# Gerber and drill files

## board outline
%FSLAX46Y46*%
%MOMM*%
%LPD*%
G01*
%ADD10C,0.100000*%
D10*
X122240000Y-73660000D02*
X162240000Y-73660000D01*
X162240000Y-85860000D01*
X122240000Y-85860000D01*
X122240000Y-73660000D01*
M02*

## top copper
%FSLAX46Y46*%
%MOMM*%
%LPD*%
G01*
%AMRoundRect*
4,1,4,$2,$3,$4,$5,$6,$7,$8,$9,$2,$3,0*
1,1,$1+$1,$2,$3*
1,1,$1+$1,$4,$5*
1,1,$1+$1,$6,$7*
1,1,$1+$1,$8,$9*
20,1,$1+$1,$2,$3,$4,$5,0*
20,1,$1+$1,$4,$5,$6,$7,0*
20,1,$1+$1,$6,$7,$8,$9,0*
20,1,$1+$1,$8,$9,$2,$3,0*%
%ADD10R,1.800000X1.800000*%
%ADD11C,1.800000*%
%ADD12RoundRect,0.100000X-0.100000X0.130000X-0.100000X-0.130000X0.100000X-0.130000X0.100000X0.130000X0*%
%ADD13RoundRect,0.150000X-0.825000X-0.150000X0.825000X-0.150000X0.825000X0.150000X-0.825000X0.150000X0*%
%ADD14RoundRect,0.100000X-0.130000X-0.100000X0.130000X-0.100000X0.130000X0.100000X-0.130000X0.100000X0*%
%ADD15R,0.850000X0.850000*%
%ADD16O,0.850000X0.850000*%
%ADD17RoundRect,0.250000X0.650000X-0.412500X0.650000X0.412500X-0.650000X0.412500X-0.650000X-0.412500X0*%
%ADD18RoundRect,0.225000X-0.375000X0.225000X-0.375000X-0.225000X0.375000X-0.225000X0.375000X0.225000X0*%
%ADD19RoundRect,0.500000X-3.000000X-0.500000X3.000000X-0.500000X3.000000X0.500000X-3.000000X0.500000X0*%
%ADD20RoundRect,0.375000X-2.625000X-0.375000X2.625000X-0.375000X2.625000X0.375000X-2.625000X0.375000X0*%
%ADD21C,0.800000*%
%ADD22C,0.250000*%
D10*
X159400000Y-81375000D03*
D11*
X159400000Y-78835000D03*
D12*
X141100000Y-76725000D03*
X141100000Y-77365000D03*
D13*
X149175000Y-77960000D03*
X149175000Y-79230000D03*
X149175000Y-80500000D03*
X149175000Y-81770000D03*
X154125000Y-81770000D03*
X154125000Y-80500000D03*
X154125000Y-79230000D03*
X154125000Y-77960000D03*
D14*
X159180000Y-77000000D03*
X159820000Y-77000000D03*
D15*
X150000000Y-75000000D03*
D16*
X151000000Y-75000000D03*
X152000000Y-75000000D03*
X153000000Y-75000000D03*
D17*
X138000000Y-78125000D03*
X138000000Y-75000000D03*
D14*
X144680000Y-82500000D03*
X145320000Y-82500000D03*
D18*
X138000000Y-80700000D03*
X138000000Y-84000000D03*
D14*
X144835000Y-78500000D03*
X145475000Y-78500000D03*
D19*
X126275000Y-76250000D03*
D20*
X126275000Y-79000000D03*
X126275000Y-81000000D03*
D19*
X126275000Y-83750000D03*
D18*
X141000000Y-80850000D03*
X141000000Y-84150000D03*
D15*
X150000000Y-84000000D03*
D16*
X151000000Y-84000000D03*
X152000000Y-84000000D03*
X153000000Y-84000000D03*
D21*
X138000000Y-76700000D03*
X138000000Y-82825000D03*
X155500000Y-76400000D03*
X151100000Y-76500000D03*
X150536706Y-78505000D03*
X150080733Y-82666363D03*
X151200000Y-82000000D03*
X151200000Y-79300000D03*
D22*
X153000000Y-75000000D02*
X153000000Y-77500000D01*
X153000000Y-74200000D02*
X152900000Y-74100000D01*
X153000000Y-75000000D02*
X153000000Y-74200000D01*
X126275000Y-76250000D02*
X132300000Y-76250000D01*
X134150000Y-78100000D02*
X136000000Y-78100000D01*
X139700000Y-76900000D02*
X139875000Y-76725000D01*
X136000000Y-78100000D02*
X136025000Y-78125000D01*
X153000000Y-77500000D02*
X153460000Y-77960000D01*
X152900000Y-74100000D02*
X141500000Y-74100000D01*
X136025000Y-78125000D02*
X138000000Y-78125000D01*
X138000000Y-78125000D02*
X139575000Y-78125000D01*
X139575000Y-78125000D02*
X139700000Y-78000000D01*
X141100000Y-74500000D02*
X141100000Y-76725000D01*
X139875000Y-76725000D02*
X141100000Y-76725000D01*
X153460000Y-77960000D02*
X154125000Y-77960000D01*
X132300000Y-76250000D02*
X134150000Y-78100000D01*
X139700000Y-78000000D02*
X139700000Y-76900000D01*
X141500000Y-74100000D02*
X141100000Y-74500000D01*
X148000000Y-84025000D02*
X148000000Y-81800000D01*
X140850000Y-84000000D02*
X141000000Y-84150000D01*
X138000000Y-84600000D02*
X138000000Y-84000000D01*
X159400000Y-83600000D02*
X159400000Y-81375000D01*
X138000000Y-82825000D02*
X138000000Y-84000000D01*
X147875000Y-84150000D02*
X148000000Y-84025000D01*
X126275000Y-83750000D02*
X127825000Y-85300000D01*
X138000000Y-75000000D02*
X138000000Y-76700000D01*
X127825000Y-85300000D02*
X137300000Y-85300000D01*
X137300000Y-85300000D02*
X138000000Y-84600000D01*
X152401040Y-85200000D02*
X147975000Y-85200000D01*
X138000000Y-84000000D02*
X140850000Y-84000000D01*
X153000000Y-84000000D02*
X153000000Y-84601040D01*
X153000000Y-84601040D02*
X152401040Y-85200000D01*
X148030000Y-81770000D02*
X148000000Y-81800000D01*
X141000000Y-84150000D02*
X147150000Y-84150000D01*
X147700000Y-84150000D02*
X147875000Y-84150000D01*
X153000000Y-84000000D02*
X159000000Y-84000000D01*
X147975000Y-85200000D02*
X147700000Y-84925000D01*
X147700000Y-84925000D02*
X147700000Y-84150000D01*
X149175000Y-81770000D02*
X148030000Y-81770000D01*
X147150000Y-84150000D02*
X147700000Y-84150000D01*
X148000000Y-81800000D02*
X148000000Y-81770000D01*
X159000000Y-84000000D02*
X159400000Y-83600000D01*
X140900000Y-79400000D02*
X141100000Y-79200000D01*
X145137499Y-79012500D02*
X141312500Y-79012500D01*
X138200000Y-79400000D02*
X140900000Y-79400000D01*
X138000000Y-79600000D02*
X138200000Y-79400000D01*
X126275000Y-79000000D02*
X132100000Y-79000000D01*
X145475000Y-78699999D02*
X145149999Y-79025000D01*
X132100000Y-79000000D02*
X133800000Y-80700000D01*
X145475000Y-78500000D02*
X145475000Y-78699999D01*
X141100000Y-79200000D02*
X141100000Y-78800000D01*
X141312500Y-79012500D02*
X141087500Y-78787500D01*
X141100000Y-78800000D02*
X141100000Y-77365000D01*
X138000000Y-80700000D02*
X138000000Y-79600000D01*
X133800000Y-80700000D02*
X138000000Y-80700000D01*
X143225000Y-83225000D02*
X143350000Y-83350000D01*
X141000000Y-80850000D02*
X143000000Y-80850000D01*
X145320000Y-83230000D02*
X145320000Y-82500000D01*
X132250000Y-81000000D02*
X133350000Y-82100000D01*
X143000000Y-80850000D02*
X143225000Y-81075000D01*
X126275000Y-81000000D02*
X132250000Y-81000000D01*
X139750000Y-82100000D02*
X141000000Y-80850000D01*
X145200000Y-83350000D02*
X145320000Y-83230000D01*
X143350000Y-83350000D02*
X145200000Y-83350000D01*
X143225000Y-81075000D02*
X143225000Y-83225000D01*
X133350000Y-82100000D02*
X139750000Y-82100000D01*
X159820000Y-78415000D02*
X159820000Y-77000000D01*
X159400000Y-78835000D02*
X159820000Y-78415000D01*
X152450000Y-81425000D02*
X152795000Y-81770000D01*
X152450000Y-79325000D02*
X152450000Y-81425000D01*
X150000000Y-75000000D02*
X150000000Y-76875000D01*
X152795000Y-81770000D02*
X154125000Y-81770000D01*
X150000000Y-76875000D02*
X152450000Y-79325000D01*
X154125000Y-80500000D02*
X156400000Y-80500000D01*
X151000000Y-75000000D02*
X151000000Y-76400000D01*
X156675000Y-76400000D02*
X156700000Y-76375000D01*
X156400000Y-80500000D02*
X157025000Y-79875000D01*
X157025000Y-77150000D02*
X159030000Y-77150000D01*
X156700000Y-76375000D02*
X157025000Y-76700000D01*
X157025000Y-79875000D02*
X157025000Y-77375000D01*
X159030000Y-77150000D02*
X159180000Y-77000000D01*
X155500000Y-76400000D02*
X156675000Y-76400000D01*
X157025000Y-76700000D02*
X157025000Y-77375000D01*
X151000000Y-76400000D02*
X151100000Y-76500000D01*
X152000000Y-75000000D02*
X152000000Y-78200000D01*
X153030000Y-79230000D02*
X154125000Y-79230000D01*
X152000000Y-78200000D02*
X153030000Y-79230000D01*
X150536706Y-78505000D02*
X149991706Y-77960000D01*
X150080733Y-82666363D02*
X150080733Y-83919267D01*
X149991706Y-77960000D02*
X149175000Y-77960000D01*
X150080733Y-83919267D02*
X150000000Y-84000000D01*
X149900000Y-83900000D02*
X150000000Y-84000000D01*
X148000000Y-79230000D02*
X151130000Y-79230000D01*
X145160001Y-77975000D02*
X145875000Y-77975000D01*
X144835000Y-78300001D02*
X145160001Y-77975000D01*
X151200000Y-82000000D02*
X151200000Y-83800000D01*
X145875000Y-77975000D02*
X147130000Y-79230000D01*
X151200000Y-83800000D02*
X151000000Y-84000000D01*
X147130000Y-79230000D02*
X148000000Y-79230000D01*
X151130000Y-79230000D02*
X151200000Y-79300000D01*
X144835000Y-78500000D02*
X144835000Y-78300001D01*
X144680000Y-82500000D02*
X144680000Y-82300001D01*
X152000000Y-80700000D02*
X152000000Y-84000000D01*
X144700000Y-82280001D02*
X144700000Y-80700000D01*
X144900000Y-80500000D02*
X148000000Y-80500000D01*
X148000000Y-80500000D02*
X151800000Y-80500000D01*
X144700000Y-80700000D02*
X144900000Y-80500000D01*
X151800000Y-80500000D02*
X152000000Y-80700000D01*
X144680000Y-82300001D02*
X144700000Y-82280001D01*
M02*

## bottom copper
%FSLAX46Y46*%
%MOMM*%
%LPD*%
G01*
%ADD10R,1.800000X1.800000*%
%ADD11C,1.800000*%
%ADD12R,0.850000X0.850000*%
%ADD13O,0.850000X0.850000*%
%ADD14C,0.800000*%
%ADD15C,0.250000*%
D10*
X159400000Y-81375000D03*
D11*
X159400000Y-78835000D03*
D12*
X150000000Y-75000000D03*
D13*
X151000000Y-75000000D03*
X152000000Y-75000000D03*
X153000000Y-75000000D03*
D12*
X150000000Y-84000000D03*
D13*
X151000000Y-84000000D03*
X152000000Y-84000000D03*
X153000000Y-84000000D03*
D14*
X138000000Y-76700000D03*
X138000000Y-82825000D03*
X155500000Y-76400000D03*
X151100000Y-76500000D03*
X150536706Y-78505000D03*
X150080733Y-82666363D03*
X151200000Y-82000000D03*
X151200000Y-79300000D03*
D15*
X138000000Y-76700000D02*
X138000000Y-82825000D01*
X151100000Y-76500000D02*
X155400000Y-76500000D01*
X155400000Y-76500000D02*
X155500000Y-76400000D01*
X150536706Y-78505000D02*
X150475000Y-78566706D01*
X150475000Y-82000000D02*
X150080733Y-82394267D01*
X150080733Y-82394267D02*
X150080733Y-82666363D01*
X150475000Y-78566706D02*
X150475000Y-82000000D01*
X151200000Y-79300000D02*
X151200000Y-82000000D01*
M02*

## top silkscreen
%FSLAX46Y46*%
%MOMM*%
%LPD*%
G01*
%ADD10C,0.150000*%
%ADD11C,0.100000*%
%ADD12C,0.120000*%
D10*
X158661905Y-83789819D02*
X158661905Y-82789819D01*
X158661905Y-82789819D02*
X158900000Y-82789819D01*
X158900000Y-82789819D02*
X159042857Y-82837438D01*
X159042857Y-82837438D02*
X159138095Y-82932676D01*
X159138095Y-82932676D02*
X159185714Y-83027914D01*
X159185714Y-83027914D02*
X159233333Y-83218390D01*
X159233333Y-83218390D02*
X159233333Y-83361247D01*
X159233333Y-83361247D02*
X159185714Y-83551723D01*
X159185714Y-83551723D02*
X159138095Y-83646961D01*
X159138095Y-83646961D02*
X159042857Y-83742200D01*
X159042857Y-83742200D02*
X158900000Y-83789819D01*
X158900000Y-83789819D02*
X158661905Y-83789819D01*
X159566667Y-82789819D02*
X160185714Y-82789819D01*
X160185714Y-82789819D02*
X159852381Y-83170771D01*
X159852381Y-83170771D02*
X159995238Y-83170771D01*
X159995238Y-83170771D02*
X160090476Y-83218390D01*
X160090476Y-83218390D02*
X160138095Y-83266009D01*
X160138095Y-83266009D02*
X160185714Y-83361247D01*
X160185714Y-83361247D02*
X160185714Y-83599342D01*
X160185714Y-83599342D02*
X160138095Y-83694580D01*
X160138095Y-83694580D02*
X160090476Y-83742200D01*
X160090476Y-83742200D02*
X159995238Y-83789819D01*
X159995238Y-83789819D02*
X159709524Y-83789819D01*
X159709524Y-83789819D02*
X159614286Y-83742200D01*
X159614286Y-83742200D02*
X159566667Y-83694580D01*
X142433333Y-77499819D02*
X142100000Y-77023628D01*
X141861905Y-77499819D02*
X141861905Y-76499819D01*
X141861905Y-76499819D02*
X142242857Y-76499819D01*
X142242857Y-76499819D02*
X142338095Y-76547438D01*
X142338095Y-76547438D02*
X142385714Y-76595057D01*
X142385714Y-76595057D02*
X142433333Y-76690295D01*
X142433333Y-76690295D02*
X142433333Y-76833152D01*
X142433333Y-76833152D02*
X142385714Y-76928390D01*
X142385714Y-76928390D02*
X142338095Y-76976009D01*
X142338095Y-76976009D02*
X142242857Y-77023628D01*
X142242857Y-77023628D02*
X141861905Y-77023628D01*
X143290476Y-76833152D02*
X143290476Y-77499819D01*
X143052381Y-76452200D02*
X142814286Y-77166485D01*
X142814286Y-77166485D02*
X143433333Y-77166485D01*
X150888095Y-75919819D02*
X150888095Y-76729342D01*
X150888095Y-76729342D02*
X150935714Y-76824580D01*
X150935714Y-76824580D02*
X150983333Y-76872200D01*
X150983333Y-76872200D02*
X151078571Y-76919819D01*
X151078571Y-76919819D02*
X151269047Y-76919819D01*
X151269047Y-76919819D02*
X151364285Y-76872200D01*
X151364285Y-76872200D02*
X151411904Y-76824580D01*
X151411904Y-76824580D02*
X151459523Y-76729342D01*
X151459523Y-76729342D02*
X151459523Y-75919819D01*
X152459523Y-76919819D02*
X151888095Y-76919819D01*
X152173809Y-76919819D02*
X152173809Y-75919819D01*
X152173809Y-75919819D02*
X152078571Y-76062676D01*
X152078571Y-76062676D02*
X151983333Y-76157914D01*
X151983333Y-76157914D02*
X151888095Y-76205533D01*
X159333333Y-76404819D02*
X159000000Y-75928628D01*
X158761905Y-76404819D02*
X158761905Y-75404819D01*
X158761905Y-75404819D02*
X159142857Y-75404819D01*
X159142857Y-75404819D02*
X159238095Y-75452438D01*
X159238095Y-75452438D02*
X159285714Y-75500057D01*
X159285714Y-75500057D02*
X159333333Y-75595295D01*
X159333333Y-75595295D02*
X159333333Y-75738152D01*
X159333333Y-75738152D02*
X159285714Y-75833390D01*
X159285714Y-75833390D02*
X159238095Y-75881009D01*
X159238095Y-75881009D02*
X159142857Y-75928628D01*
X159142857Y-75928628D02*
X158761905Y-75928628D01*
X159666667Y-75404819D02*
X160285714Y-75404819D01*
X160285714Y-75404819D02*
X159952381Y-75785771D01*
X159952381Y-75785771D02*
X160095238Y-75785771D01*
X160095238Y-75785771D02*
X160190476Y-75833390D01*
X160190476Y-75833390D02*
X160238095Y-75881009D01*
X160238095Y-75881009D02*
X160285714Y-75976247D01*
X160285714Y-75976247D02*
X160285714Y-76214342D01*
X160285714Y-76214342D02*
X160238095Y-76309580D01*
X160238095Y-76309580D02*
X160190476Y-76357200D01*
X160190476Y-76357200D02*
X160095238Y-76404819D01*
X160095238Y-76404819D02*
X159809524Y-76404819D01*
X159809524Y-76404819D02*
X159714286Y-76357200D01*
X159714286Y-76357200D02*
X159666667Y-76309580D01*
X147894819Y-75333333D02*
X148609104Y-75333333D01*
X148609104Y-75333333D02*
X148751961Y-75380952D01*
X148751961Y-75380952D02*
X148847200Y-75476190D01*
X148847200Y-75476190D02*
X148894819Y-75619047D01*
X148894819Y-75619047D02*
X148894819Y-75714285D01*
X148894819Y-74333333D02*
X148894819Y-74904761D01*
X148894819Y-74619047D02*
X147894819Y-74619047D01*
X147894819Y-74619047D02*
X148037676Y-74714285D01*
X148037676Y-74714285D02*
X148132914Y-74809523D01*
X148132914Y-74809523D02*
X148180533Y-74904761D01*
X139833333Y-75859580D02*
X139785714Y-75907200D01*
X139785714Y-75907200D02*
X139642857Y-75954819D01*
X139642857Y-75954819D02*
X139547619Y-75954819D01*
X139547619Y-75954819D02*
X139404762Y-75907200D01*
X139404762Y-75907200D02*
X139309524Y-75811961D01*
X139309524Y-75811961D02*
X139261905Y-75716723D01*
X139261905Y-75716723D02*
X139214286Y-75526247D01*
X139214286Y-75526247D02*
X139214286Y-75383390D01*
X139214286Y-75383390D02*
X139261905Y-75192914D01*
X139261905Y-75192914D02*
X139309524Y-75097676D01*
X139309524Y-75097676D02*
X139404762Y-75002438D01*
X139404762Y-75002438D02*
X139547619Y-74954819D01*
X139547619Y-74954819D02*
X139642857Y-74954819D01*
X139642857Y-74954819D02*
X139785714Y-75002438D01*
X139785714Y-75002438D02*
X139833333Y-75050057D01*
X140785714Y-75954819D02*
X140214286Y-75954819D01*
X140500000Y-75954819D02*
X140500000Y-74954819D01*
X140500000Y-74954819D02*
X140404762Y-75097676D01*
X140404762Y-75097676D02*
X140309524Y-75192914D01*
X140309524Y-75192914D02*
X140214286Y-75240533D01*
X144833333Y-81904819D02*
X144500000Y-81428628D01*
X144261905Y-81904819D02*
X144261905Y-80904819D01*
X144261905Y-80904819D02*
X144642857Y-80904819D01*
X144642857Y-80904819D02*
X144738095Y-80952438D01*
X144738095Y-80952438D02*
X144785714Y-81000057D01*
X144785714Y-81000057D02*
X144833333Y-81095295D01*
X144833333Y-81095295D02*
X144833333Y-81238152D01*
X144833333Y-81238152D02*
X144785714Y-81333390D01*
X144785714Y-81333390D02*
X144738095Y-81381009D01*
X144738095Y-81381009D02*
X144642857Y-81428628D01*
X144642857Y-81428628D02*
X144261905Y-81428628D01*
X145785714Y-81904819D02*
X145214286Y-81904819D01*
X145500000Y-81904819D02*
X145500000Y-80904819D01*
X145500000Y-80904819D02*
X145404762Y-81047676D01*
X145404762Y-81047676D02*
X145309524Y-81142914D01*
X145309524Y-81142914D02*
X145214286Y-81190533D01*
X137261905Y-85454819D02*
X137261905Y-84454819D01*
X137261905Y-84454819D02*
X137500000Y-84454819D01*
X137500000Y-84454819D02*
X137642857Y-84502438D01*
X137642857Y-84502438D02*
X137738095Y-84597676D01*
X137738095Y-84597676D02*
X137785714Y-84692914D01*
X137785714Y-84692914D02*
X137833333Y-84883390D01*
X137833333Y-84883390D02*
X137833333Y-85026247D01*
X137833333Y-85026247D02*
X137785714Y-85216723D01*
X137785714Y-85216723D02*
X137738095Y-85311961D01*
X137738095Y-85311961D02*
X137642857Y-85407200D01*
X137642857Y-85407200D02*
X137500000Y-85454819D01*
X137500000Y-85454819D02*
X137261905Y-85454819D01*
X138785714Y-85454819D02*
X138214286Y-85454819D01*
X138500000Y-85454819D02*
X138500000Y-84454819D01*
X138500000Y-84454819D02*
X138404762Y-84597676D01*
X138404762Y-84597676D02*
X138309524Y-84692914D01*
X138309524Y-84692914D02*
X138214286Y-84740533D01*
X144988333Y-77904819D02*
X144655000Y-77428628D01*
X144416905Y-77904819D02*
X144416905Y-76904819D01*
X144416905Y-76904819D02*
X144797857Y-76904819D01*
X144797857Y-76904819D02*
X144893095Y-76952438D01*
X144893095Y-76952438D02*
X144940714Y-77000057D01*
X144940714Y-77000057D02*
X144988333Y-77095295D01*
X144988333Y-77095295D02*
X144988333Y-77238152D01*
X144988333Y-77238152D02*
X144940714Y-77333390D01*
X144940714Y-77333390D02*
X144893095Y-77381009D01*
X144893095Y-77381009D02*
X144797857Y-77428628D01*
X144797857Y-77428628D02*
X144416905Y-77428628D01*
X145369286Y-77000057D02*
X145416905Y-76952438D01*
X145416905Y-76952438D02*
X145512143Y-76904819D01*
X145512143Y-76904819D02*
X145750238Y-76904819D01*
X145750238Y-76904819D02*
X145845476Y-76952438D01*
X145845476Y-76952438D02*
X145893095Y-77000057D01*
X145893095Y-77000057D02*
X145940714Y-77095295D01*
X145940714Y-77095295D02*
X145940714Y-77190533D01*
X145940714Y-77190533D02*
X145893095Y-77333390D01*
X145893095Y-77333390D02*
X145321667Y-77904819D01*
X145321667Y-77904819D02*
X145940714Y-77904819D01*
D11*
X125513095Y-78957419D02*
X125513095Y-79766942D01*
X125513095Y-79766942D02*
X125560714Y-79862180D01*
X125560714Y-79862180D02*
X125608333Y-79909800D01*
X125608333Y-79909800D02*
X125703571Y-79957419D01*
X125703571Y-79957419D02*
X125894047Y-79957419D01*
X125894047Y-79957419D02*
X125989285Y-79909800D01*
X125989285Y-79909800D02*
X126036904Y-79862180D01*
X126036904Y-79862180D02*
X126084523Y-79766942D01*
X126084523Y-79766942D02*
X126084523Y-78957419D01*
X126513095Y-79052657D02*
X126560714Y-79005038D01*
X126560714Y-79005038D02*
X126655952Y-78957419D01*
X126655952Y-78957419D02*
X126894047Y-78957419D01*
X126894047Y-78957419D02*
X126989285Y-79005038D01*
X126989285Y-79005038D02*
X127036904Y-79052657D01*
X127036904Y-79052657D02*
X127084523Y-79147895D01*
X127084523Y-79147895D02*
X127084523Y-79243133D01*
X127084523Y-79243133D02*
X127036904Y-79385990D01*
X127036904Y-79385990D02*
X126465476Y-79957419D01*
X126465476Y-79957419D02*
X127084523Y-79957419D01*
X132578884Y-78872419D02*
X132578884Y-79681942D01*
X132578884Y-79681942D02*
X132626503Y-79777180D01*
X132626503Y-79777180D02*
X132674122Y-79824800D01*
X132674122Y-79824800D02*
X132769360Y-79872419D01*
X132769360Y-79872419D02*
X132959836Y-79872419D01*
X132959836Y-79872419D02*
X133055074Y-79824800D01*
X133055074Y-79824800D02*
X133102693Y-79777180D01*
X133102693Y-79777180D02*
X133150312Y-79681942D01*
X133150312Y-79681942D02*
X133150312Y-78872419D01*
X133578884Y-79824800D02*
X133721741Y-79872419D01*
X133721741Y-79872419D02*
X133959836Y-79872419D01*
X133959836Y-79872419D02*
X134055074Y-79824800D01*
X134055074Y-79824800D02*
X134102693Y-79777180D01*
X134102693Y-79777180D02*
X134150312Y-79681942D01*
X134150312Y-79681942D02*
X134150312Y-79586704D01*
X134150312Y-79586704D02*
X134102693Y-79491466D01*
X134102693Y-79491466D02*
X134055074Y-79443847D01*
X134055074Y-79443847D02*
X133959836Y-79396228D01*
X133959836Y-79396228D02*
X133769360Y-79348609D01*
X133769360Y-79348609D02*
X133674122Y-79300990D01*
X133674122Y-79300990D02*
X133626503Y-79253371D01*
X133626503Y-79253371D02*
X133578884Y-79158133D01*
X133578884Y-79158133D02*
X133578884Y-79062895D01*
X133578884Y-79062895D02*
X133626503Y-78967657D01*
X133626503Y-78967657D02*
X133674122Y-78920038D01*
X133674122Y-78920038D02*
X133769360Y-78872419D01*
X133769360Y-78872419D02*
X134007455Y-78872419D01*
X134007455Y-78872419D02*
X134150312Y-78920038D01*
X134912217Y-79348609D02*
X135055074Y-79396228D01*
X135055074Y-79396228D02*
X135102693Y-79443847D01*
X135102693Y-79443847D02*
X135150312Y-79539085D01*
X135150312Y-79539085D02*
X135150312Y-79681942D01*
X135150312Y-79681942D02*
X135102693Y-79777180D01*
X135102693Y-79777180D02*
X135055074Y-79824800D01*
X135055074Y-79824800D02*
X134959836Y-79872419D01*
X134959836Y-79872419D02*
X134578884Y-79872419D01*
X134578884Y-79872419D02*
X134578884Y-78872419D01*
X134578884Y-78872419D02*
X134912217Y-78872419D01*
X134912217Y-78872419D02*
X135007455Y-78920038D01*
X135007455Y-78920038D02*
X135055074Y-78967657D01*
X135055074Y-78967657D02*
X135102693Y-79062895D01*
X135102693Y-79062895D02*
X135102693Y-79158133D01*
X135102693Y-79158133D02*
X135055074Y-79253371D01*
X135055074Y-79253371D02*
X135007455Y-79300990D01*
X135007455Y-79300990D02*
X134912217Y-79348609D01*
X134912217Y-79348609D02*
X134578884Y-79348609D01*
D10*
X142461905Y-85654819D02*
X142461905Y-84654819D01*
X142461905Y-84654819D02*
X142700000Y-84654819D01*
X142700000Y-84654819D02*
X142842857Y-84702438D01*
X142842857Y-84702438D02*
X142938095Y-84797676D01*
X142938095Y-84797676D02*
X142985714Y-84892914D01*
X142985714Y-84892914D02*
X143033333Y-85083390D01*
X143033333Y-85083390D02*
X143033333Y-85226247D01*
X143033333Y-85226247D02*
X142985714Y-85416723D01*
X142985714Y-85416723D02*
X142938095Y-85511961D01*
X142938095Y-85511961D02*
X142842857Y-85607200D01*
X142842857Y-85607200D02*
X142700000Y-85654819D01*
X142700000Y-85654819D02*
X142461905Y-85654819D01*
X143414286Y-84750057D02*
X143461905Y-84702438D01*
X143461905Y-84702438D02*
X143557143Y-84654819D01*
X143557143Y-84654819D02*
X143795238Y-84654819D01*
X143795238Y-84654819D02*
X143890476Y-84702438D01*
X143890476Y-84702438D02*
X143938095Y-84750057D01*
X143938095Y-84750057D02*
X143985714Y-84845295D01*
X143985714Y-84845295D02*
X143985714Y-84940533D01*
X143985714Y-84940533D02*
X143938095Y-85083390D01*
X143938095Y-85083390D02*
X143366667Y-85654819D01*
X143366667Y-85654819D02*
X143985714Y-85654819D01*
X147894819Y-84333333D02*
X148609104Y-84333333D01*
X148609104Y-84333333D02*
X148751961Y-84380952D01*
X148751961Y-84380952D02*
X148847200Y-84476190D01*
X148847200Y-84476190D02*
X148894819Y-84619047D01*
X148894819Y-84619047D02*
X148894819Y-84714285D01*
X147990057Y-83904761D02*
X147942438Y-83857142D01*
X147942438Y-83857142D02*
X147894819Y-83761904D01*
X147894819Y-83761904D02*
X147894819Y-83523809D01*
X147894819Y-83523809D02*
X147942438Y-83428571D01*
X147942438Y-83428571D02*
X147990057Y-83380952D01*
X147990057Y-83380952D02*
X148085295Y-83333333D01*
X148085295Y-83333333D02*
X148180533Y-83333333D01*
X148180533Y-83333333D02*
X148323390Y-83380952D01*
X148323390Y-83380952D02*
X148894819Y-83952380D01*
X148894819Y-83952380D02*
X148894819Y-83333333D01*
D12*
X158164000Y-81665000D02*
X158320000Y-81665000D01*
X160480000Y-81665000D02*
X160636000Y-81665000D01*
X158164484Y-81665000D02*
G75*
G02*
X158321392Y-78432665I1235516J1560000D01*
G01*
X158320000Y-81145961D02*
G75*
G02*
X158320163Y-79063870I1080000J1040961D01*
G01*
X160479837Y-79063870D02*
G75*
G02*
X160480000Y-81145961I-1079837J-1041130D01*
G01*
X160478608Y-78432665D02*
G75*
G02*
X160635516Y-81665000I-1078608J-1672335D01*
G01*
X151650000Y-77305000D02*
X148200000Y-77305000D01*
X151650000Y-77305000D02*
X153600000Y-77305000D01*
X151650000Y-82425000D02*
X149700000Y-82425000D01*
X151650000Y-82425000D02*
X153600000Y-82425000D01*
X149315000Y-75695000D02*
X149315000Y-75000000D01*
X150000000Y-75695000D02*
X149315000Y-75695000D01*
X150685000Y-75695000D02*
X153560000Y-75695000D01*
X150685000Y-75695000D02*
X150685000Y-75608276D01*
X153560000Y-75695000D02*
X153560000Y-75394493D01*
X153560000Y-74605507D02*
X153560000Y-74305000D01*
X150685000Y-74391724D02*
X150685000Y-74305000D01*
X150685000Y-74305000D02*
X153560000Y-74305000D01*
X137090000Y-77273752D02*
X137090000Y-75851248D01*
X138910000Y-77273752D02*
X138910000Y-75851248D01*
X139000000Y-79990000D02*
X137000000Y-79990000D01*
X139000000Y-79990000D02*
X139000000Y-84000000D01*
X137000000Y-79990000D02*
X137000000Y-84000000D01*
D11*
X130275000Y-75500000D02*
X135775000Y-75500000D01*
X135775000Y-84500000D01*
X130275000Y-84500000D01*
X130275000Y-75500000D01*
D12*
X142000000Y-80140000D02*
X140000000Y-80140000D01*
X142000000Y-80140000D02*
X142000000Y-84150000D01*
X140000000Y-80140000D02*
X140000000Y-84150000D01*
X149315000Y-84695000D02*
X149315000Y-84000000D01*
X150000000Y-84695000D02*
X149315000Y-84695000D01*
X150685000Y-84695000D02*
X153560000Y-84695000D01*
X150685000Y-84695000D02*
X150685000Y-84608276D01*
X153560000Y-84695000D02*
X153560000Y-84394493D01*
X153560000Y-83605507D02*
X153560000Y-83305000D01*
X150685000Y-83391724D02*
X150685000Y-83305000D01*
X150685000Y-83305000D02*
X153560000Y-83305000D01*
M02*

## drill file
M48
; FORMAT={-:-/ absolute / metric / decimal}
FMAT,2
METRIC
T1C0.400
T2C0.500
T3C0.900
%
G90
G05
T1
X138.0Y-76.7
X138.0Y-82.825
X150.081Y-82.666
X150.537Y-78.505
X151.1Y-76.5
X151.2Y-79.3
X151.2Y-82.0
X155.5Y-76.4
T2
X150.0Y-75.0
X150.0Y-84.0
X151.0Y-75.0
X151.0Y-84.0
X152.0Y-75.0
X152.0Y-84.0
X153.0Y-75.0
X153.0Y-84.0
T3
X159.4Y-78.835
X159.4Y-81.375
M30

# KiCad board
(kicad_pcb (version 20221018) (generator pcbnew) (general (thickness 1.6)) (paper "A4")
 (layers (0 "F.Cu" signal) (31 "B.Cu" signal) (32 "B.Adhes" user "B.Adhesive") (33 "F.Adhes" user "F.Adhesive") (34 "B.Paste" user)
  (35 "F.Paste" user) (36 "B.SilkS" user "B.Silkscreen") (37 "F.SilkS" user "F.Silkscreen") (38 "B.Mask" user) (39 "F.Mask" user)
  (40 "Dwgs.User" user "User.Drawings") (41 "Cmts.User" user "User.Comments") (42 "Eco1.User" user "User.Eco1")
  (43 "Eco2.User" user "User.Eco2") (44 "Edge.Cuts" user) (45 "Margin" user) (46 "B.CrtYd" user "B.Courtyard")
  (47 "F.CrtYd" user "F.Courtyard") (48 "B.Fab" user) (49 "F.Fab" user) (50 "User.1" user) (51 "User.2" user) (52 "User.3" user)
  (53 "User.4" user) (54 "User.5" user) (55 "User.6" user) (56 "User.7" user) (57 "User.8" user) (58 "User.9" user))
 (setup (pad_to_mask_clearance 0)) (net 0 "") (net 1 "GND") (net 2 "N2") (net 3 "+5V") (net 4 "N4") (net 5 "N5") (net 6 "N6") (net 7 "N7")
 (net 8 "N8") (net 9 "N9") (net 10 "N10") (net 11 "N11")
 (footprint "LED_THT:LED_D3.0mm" (layer "F.Cu") (at 159.4 81.375 90)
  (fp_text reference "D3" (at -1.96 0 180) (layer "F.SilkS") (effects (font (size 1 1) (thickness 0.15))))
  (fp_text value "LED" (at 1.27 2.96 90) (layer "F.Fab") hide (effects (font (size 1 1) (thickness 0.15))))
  (fp_line (start -0.29 -1.236) (end -0.29 -1.08) (stroke (width 0.12) (type solid)) (layer "F.SilkS"))
  (fp_line (start -0.29 1.08) (end -0.29 1.236) (stroke (width 0.12) (type solid)) (layer "F.SilkS"))
  (fp_arc (start -0.29 -1.235516) (mid 1.366487 -1.987659) (end 2.942335 -1.078608) (stroke (width 0.12) (type solid)) (layer "F.SilkS"))
  (fp_arc (start 0.229039 -1.08) (mid 1.270117 -1.5) (end 2.31113 -1.079837) (stroke (width 0.12) (type solid)) (layer "F.SilkS"))
  (fp_arc (start 2.31113 1.079837) (mid 1.270117 1.5) (end 0.229039 1.08) (stroke (width 0.12) (type solid)) (layer "F.SilkS"))
  (fp_arc (start 2.942335 1.078608) (mid 1.366487 1.987659) (end -0.29 1.235516) (stroke (width 0.12) (type solid)) (layer "F.SilkS"))
  (pad "1" thru_hole rect (at 0 0 90) (size 1.8 1.8) (drill 0.9) (layers "*.Cu" "*.Mask") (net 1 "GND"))
  (pad "2" thru_hole circle (at 2.54 0 90) (size 1.8 1.8) (drill 0.9) (layers "*.Cu" "*.Mask") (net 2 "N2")))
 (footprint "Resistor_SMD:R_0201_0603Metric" (layer "F.Cu") (at 141.1 77.045 -90)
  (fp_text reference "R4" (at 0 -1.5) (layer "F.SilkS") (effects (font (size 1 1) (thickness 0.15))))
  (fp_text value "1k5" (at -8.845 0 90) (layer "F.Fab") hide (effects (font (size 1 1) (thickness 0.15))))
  (pad "" smd roundrect (at -0.345 0 270) (size 0.318 0.36) (layers "F.Paste") (roundrect_rratio 0.25))
  (pad "" smd roundrect (at 0.345 0 270) (size 0.318 0.36) (layers "F.Paste") (roundrect_rratio 0.25))
  (pad "1" smd roundrect (at -0.32 0 270) (size 0.46 0.4) (layers "F.Cu" "F.Mask") (roundrect_rratio 0.25) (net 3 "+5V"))
  (pad "2" smd roundrect (at 0.32 0 270) (size 0.46 0.4) (layers "F.Cu" "F.Mask") (roundrect_rratio 0.25) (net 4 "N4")))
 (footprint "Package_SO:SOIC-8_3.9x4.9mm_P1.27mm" (layer "F.Cu") (at 151.65 79.865)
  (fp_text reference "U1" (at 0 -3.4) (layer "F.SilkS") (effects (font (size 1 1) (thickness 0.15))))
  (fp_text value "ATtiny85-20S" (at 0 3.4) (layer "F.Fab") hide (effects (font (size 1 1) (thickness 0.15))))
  (fp_line (start 0 -2.56) (end -3.45 -2.56) (stroke (width 0.12) (type solid)) (layer "F.SilkS"))
  (fp_line (start 0 -2.56) (end 1.95 -2.56) (stroke (width 0.12) (type solid)) (layer "F.SilkS"))
  (fp_line (start 0 2.56) (end -1.95 2.56) (stroke (width 0.12) (type solid)) (layer "F.SilkS"))
  (fp_line (start 0 2.56) (end 1.95 2.56) (stroke (width 0.12) (type solid)) (layer "F.SilkS"))
  (pad "1" smd roundrect (at -2.475 -1.905) (size 1.95 0.6) (layers "F.Cu" "F.Paste" "F.Mask") (roundrect_rratio 0.25) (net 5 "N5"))
  (pad "2" smd roundrect (at -2.475 -0.635) (size 1.95 0.6) (layers "F.Cu" "F.Paste" "F.Mask") (roundrect_rratio 0.25) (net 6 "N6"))
  (pad "3" smd roundrect (at -2.475 0.635) (size 1.95 0.6) (layers "F.Cu" "F.Paste" "F.Mask") (roundrect_rratio 0.25) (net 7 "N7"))
  (pad "4" smd roundrect (at -2.475 1.905) (size 1.95 0.6) (layers "F.Cu" "F.Paste" "F.Mask") (roundrect_rratio 0.25) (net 1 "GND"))
  (pad "5" smd roundrect (at 2.475 1.905) (size 1.95 0.6) (layers "F.Cu" "F.Paste" "F.Mask") (roundrect_rratio 0.25) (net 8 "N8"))
  (pad "6" smd roundrect (at 2.475 0.635) (size 1.95 0.6) (layers "F.Cu" "F.Paste" "F.Mask") (roundrect_rratio 0.25) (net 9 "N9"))
  (pad "7" smd roundrect (at 2.475 -0.635) (size 1.95 0.6) (layers "F.Cu" "F.Paste" "F.Mask") (roundrect_rratio 0.25) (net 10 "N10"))
  (pad "8" smd roundrect (at 2.475 -1.905) (size 1.95 0.6) (layers "F.Cu" "F.Paste" "F.Mask") (roundrect_rratio 0.25) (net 3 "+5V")))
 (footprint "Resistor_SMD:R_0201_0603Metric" (layer "F.Cu") (at 159.5 77)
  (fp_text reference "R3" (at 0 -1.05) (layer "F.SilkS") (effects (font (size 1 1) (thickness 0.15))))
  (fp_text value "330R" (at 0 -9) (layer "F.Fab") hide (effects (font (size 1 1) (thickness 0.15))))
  (pad "" smd roundrect (at -0.345 0) (size 0.318 0.36) (layers "F.Paste") (roundrect_rratio 0.25))
  (pad "" smd roundrect (at 0.345 0) (size 0.318 0.36) (layers "F.Paste") (roundrect_rratio 0.25))
  (pad "1" smd roundrect (at -0.32 0) (size 0.46 0.4) (layers "F.Cu" "F.Mask") (roundrect_rratio 0.25) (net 9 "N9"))
  (pad "2" smd roundrect (at 0.32 0) (size 0.46 0.4) (layers "F.Cu" "F.Mask") (roundrect_rratio 0.25) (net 2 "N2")))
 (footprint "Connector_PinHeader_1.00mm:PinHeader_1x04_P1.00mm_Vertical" (layer "F.Cu") (at 150 75 90)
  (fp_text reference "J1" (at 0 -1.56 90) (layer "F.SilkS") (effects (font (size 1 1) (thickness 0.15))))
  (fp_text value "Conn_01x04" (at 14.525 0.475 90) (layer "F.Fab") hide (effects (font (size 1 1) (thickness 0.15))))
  (fp_line (start -0.695 -0.685) (end 0 -0.685) (stroke (width 0.12) (type solid)) (layer "F.SilkS"))
  (fp_line (start -0.695 0) (end -0.695 -0.685) (stroke (width 0.12) (type solid)) (layer "F.SilkS"))
  (fp_line (start -0.695 0.685) (end -0.695 3.56) (stroke (width 0.12) (type solid)) (layer "F.SilkS"))
  (fp_line (start -0.695 0.685) (end -0.608276 0.685) (stroke (width 0.12) (type solid)) (layer "F.SilkS"))
  (fp_line (start -0.695 3.56) (end -0.394493 3.56) (stroke (width 0.12) (type solid)) (layer "F.SilkS"))
  (fp_line (start 0.394493 3.56) (end 0.695 3.56) (stroke (width 0.12) (type solid)) (layer "F.SilkS"))
  (fp_line (start 0.608276 0.685) (end 0.695 0.685) (stroke (width 0.12) (type solid)) (layer "F.SilkS"))
  (fp_line (start 0.695 0.685) (end 0.695 3.56) (stroke (width 0.12) (type solid)) (layer "F.SilkS"))
  (pad "1" thru_hole rect (at 0 0 90) (size 0.85 0.85) (drill 0.5) (layers "*.Cu" "*.Mask") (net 8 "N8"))
  (pad "2" thru_hole oval (at 0 1 90) (size 0.85 0.85) (drill 0.5) (layers "*.Cu" "*.Mask") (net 9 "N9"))
  (pad "3" thru_hole oval (at 0 2 90) (size 0.85 0.85) (drill 0.5) (layers "*.Cu" "*.Mask") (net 10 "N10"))
  (pad "4" thru_hole oval (at 0 3 90) (size 0.85 0.85) (drill 0.5) (layers "*.Cu" "*.Mask") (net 3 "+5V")))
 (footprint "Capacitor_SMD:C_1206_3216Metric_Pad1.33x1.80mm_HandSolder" (layer "F.Cu") (at 138 76.5625 90)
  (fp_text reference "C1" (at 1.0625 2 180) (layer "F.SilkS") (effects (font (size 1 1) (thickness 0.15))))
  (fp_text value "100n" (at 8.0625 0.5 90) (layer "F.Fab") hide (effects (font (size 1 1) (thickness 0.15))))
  (fp_line (start -0.711252 -0.91) (end 0.711252 -0.91) (stroke (width 0.12) (type solid)) (layer "F.SilkS"))
  (fp_line (start -0.711252 0.91) (end 0.711252 0.91) (stroke (width 0.12) (type solid)) (layer "F.SilkS"))
  (pad "1" smd roundrect (at -1.5625 0 90) (size 1.325 1.8) (layers "F.Cu" "F.Paste" "F.Mask") (roundrect_rratio 0.188679) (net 3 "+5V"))
  (pad "2" smd roundrect (at 1.5625 0 90) (size 1.325 1.8) (layers "F.Cu" "F.Paste" "F.Mask") (roundrect_rratio 0.188679) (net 1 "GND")))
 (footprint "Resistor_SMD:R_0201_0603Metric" (layer "F.Cu") (at 145 82.5)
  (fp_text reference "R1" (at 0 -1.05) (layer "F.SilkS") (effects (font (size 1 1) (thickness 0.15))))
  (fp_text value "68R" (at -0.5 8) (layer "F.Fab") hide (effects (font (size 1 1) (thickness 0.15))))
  (pad "" smd roundrect (at -0.345 0) (size 0.318 0.36) (layers "F.Paste") (roundrect_rratio 0.25))
  (pad "" smd roundrect (at 0.345 0) (size 0.318 0.36) (layers "F.Paste") (roundrect_rratio 0.25))
  (pad "1" smd roundrect (at -0.32 0) (size 0.46 0.4) (layers "F.Cu" "F.Mask") (roundrect_rratio 0.25) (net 7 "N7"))
  (pad "2" smd roundrect (at 0.32 0) (size 0.46 0.4) (layers "F.Cu" "F.Mask") (roundrect_rratio 0.25) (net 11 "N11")))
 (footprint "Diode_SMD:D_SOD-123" (layer "F.Cu") (at 138 82.35 -90)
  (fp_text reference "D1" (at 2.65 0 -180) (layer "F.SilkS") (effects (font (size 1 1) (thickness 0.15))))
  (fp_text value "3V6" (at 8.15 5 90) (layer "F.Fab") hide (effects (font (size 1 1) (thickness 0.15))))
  (fp_line (start -2.36 -1) (end -2.36 1) (stroke (width 0.12) (type solid)) (layer "F.SilkS"))
  (fp_line (start -2.36 -1) (end 1.65 -1) (stroke (width 0.12) (type solid)) (layer "F.SilkS"))
  (fp_line (start -2.36 1) (end 1.65 1) (stroke (width 0.12) (type solid)) (layer "F.SilkS"))
  (pad "1" smd roundrect (at -1.65 0 270) (size 0.9 1.2) (layers "F.Cu" "F.Paste" "F.Mask") (roundrect_rratio 0.25) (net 4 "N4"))
  (pad "2" smd roundrect (at 1.65 0 270) (size 0.9 1.2) (layers "F.Cu" "F.Paste" "F.Mask") (roundrect_rratio 0.25) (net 1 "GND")))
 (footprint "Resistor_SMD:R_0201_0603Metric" (layer "F.Cu") (at 145.155 78.5)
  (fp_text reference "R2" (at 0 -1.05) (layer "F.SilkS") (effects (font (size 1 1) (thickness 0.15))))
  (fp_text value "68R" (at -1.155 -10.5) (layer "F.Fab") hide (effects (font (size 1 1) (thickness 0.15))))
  (pad "" smd roundrect (at -0.345 0) (size 0.318 0.36) (layers "F.Paste") (roundrect_rratio 0.25))
  (pad "" smd roundrect (at 0.345 0) (size 0.318 0.36) (layers "F.Paste") (roundrect_rratio 0.25))
  (pad "1" smd roundrect (at -0.32 0) (size 0.46 0.4) (layers "F.Cu" "F.Mask") (roundrect_rratio 0.25) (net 6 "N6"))
  (pad "2" smd roundrect (at 0.32 0) (size 0.46 0.4) (layers "F.Cu" "F.Mask") (roundrect_rratio 0.25) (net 4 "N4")))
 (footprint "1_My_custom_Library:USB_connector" (layer "F.Cu") (at 126.275 80)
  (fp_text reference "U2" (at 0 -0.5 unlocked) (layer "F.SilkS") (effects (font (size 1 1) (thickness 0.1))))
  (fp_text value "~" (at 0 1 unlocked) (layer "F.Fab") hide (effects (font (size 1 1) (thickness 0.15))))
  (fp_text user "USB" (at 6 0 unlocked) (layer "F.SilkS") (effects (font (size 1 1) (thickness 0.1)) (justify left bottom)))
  (fp_rect (start 4 -4.5) (end 9.5 4.5) (stroke (width 0.1) (type default)) (fill none) (layer "F.SilkS"))
  (pad "1" smd roundrect (at 0 -3.75) (size 7 2) (layers "F.Cu" "F.Paste" "F.Mask") (roundrect_rratio 0.25) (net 3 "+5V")
   (thermal_bridge_angle 45))
  (pad "2" smd roundrect (at 0 -1) (size 6 1.5) (layers "F.Cu" "F.Paste" "F.Mask") (roundrect_rratio 0.25) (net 4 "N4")
   (thermal_bridge_angle 45))
  (pad "3" smd roundrect (at 0 1) (size 6 1.5) (layers "F.Cu" "F.Paste" "F.Mask") (roundrect_rratio 0.25) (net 11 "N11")
   (thermal_bridge_angle 45))
  (pad "4" smd roundrect (at 0 3.75) (size 7 2) (layers "F.Cu" "F.Paste" "F.Mask") (roundrect_rratio 0.25) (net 1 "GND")
   (thermal_bridge_angle 45)))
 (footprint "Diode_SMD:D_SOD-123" (layer "F.Cu") (at 141 82.5 -90)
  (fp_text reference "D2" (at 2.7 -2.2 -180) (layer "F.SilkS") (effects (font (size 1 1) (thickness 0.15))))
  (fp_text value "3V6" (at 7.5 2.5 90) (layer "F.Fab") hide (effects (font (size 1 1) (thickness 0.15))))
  (fp_line (start -2.36 -1) (end -2.36 1) (stroke (width 0.12) (type solid)) (layer "F.SilkS"))
  (fp_line (start -2.36 -1) (end 1.65 -1) (stroke (width 0.12) (type solid)) (layer "F.SilkS"))
  (fp_line (start -2.36 1) (end 1.65 1) (stroke (width 0.12) (type solid)) (layer "F.SilkS"))
  (pad "1" smd roundrect (at -1.65 0 270) (size 0.9 1.2) (layers "F.Cu" "F.Paste" "F.Mask") (roundrect_rratio 0.25) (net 11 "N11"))
  (pad "2" smd roundrect (at 1.65 0 270) (size 0.9 1.2) (layers "F.Cu" "F.Paste" "F.Mask") (roundrect_rratio 0.25) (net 1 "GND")))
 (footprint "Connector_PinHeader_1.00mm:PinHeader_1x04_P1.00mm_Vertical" (layer "F.Cu") (at 150 84 90)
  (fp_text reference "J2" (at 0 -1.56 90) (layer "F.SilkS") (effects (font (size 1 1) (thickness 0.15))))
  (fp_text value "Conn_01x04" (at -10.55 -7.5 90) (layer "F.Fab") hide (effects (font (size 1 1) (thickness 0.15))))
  (fp_line (start -0.695 -0.685) (end 0 -0.685) (stroke (width 0.12) (type solid)) (layer "F.SilkS"))
  (fp_line (start -0.695 0) (end -0.695 -0.685) (stroke (width 0.12) (type solid)) (layer "F.SilkS"))
  (fp_line (start -0.695 0.685) (end -0.695 3.56) (stroke (width 0.12) (type solid)) (layer "F.SilkS"))
  (fp_line (start -0.695 0.685) (end -0.608276 0.685) (stroke (width 0.12) (type solid)) (layer "F.SilkS"))
  (fp_line (start -0.695 3.56) (end -0.394493 3.56) (stroke (width 0.12) (type solid)) (layer "F.SilkS"))
  (fp_line (start 0.394493 3.56) (end 0.695 3.56) (stroke (width 0.12) (type solid)) (layer "F.SilkS"))
  (fp_line (start 0.608276 0.685) (end 0.695 0.685) (stroke (width 0.12) (type solid)) (layer "F.SilkS"))
  (fp_line (start 0.695 0.685) (end 0.695 3.56) (stroke (width 0.12) (type solid)) (layer "F.SilkS"))
  (pad "1" thru_hole rect (at 0 0 90) (size 0.85 0.85) (drill 0.5) (layers "*.Cu" "*.Mask") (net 5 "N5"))
  (pad "2" thru_hole oval (at 0 1 90) (size 0.85 0.85) (drill 0.5) (layers "*.Cu" "*.Mask") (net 6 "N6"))
  (pad "3" thru_hole oval (at 0 2 90) (size 0.85 0.85) (drill 0.5) (layers "*.Cu" "*.Mask") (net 7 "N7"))
  (pad "4" thru_hole oval (at 0 3 90) (size 0.85 0.85) (drill 0.5) (layers "*.Cu" "*.Mask") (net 1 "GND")))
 (gr_rect (start 122.24 73.66) (end 162.24 85.86) (stroke (width 0.1) (type default)) (fill none) (layer "Edge.Cuts"))
 (segment (start 153 75) (end 153 77.5) (width 0.25) (layer "F.Cu") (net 3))
 (segment (start 153 74.2) (end 152.9 74.1) (width 0.25) (layer "F.Cu") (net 3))
 (segment (start 153 75) (end 153 74.2) (width 0.25) (layer "F.Cu") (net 3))
 (segment (start 126.275 76.25) (end 132.3 76.25) (width 0.25) (layer "F.Cu") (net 3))
 (segment (start 134.15 78.1) (end 136 78.1) (width 0.25) (layer "F.Cu") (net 3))
 (segment (start 139.7 76.9) (end 139.875 76.725) (width 0.25) (layer "F.Cu") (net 3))
 (segment (start 136 78.1) (end 136.025 78.125) (width 0.25) (layer "F.Cu") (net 3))
 (segment (start 153 77.5) (end 153.46 77.96) (width 0.25) (layer "F.Cu") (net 3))
 (segment (start 152.9 74.1) (end 141.5 74.1) (width 0.25) (layer "F.Cu") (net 3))
 (segment (start 136.025 78.125) (end 138 78.125) (width 0.25) (layer "F.Cu") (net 3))
 (segment (start 138 78.125) (end 139.575 78.125) (width 0.25) (layer "F.Cu") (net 3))
 (segment (start 139.575 78.125) (end 139.7 78) (width 0.25) (layer "F.Cu") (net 3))
 (segment (start 141.1 74.5) (end 141.1 76.725) (width 0.25) (layer "F.Cu") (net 3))
 (segment (start 139.875 76.725) (end 141.1 76.725) (width 0.25) (layer "F.Cu") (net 3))
 (segment (start 153.46 77.96) (end 154.125 77.96) (width 0.25) (layer "F.Cu") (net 3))
 (segment (start 132.3 76.25) (end 134.15 78.1) (width 0.25) (layer "F.Cu") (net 3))
 (segment (start 139.7 78) (end 139.7 76.9) (width 0.25) (layer "F.Cu") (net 3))
 (segment (start 141.5 74.1) (end 141.1 74.5) (width 0.25) (layer "F.Cu") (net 3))
 (segment (start 148 84.025) (end 148 81.8) (width 0.25) (layer "F.Cu") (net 1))
 (segment (start 140.85 84) (end 141 84.15) (width 0.25) (layer "F.Cu") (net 1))
 (segment (start 138 84.6) (end 138 84) (width 0.25) (layer "F.Cu") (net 1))
 (segment (start 159.4 83.6) (end 159.4 81.375) (width 0.25) (layer "F.Cu") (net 1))
 (segment (start 138 82.825) (end 138 84) (width 0.25) (layer "F.Cu") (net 1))
 (segment (start 147.875 84.15) (end 148 84.025) (width 0.25) (layer "F.Cu") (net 1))
 (segment (start 126.275 83.75) (end 127.825 85.3) (width 0.25) (layer "F.Cu") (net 1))
 (segment (start 138 75) (end 138 76.7) (width 0.25) (layer "F.Cu") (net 1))
 (segment (start 127.825 85.3) (end 137.3 85.3) (width 0.25) (layer "F.Cu") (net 1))
 (segment (start 137.3 85.3) (end 138 84.6) (width 0.25) (layer "F.Cu") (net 1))
 (segment (start 152.40104 85.2) (end 147.975 85.2) (width 0.25) (layer "F.Cu") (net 1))
 (segment (start 138 84) (end 140.85 84) (width 0.25) (layer "F.Cu") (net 1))
 (segment (start 153 84) (end 153 84.60104) (width 0.25) (layer "F.Cu") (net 1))
 (segment (start 153 84.60104) (end 152.40104 85.2) (width 0.25) (layer "F.Cu") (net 1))
 (segment (start 148.03 81.77) (end 148 81.8) (width 0.25) (layer "F.Cu") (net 1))
 (segment (start 141 84.15) (end 147.15 84.15) (width 0.25) (layer "F.Cu") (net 1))
 (segment (start 147.7 84.15) (end 147.875 84.15) (width 0.25) (layer "F.Cu") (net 1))
 (segment (start 153 84) (end 159 84) (width 0.25) (layer "F.Cu") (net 1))
 (segment (start 147.975 85.2) (end 147.7 84.925) (width 0.25) (layer "F.Cu") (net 1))
 (segment (start 147.7 84.925) (end 147.7 84.15) (width 0.25) (layer "F.Cu") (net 1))
 (segment (start 149.175 81.77) (end 148.03 81.77) (width 0.25) (layer "F.Cu") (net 1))
 (segment (start 147.15 84.15) (end 147.7 84.15) (width 0.25) (layer "F.Cu") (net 1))
 (segment (start 148 81.8) (end 148 81.77) (width 0.25) (layer "F.Cu") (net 1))
 (segment (start 159 84) (end 159.4 83.6) (width 0.25) (layer "F.Cu") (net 1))
 (via (at 138 76.7) (size 0.8) (drill 0.4) (layers "F.Cu" "B.Cu") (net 1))
 (via (at 138 82.825) (size 0.8) (drill 0.4) (layers "F.Cu" "B.Cu") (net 1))
 (segment (start 138 76.7) (end 138 82.825) (width 0.25) (layer "B.Cu") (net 1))
 (segment (start 140.9 79.4) (end 141.1 79.2) (width 0.25) (layer "F.Cu") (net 4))
 (segment (start 145.137499 79.0125) (end 141.3125 79.0125) (width 0.25) (layer "F.Cu") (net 4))
 (segment (start 138.2 79.4) (end 140.9 79.4) (width 0.25) (layer "F.Cu") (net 4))
 (segment (start 138 79.6) (end 138.2 79.4) (width 0.25) (layer "F.Cu") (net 4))
 (segment (start 126.275 79) (end 132.1 79) (width 0.25) (layer "F.Cu") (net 4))
 (segment (start 145.475 78.699999) (end 145.149999 79.025) (width 0.25) (layer "F.Cu") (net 4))
 (segment (start 132.1 79) (end 133.8 80.7) (width 0.25) (layer "F.Cu") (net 4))
 (segment (start 145.475 78.5) (end 145.475 78.699999) (width 0.25) (layer "F.Cu") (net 4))
 (segment (start 141.1 79.2) (end 141.1 78.8) (width 0.25) (layer "F.Cu") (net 4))
 (segment (start 141.3125 79.0125) (end 141.0875 78.7875) (width 0.25) (layer "F.Cu") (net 4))
 (segment (start 141.1 78.8) (end 141.1 77.365) (width 0.25) (layer "F.Cu") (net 4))
 (segment (start 138 80.7) (end 138 79.6) (width 0.25) (layer "F.Cu") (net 4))
 (segment (start 133.8 80.7) (end 138 80.7) (width 0.25) (layer "F.Cu") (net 4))
 (segment (start 143.225 83.225) (end 143.35 83.35) (width 0.25) (layer "F.Cu") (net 11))
 (segment (start 141 80.85) (end 143 80.85) (width 0.25) (layer "F.Cu") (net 11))
 (segment (start 145.32 83.23) (end 145.32 82.5) (width 0.25) (layer "F.Cu") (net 11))
 (segment (start 132.25 81) (end 133.35 82.1) (width 0.25) (layer "F.Cu") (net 11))
 (segment (start 143 80.85) (end 143.225 81.075) (width 0.25) (layer "F.Cu") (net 11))
 (segment (start 126.275 81) (end 132.25 81) (width 0.25) (layer "F.Cu") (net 11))
 (segment (start 139.75 82.1) (end 141 80.85) (width 0.25) (layer "F.Cu") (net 11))
 (segment (start 145.2 83.35) (end 145.32 83.23) (width 0.25) (layer "F.Cu") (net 11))
 (segment (start 143.35 83.35) (end 145.2 83.35) (width 0.25) (layer "F.Cu") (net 11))
 (segment (start 143.225 81.075) (end 143.225 83.225) (width 0.25) (layer "F.Cu") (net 11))
 (segment (start 133.35 82.1) (end 139.75 82.1) (width 0.25) (layer "F.Cu") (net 11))
 (segment (start 159.82 78.415) (end 159.82 77) (width 0.25) (layer "F.Cu") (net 2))
 (segment (start 159.4 78.835) (end 159.82 78.415) (width 0.25) (layer "F.Cu") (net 2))
 (segment (start 152.45 81.425) (end 152.795 81.77) (width 0.25) (layer "F.Cu") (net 8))
 (segment (start 152.45 79.325) (end 152.45 81.425) (width 0.25) (layer "F.Cu") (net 8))
 (segment (start 150 75) (end 150 76.875) (width 0.25) (layer "F.Cu") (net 8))
 (segment (start 152.795 81.77) (end 154.125 81.77) (width 0.25) (layer "F.Cu") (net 8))
 (segment (start 150 76.875) (end 152.45 79.325) (width 0.25) (layer "F.Cu") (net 8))
 (segment (start 154.125 80.5) (end 156.4 80.5) (width 0.25) (layer "F.Cu") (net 9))
 (segment (start 151 75) (end 151 76.4) (width 0.25) (layer "F.Cu") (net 9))
 (segment (start 156.675 76.4) (end 156.7 76.375) (width 0.25) (layer "F.Cu") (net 9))
 (segment (start 156.4 80.5) (end 157.025 79.875) (width 0.25) (layer "F.Cu") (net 9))
 (segment (start 157.025 77.15) (end 159.03 77.15) (width 0.25) (layer "F.Cu") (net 9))
 (segment (start 156.7 76.375) (end 157.025 76.7) (width 0.25) (layer "F.Cu") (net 9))
 (segment (start 157.025 79.875) (end 157.025 77.375) (width 0.25) (layer "F.Cu") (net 9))
 (segment (start 159.03 77.15) (end 159.18 77) (width 0.25) (layer "F.Cu") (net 9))
 (segment (start 155.5 76.4) (end 156.675 76.4) (width 0.25) (layer "F.Cu") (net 9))
 (segment (start 157.025 76.7) (end 157.025 77.375) (width 0.25) (layer "F.Cu") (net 9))
 (segment (start 151 76.4) (end 151.1 76.5) (width 0.25) (layer "F.Cu") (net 9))
 (via (at 155.5 76.4) (size 0.8) (drill 0.4) (layers "F.Cu" "B.Cu") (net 9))
 (via (at 151.1 76.5) (size 0.8) (drill 0.4) (layers "F.Cu" "B.Cu") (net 9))
 (segment (start 151.1 76.5) (end 155.4 76.5) (width 0.25) (layer "B.Cu") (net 9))
 (segment (start 155.4 76.5) (end 155.5 76.4) (width 0.25) (layer "B.Cu") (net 9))
 (segment (start 152 75) (end 152 78.2) (width 0.25) (layer "F.Cu") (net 10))
 (segment (start 153.03 79.23) (end 154.125 79.23) (width 0.25) (layer "F.Cu") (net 10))
 (segment (start 152 78.2) (end 153.03 79.23) (width 0.25) (layer "F.Cu") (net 10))
 (segment (start 150.536706 78.505) (end 149.991706 77.96) (width 0.25) (layer "F.Cu") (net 5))
 (segment (start 150.080733 82.666363) (end 150.080733 83.919267) (width 0.25) (layer "F.Cu") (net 5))
 (segment (start 149.991706 77.96) (end 149.175 77.96) (width 0.25) (layer "F.Cu") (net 5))
 (segment (start 150.080733 83.919267) (end 150 84) (width 0.25) (layer "F.Cu") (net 5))
 (segment (start 149.9 83.9) (end 150 84) (width 0.25) (layer "F.Cu") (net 5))
 (via (at 150.536706 78.505) (size 0.8) (drill 0.4) (layers "F.Cu" "B.Cu") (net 5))
 (via (at 150.080733 82.666363) (size 0.8) (drill 0.4) (layers "F.Cu" "B.Cu") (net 5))
 (segment (start 150.536706 78.505) (end 150.475 78.566706) (width 0.25) (layer "B.Cu") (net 5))
 (segment (start 150.475 82) (end 150.080733 82.394267) (width 0.25) (layer "B.Cu") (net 5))
 (segment (start 150.080733 82.394267) (end 150.080733 82.666363) (width 0.25) (layer "B.Cu") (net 5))
 (segment (start 150.475 78.566706) (end 150.475 82) (width 0.25) (layer "B.Cu") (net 5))
 (segment (start 148 79.23) (end 151.13 79.23) (width 0.25) (layer "F.Cu") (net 6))
 (segment (start 145.160001 77.975) (end 145.875 77.975) (width 0.25) (layer "F.Cu") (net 6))
 (segment (start 144.835 78.300001) (end 145.160001 77.975) (width 0.25) (layer "F.Cu") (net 6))
 (segment (start 151.2 82) (end 151.2 83.8) (width 0.25) (layer "F.Cu") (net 6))
 (segment (start 145.875 77.975) (end 147.13 79.23) (width 0.25) (layer "F.Cu") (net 6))
 (segment (start 151.2 83.8) (end 151 84) (width 0.25) (layer "F.Cu") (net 6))
 (segment (start 147.13 79.23) (end 148 79.23) (width 0.25) (layer "F.Cu") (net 6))
 (segment (start 151.13 79.23) (end 151.2 79.3) (width 0.25) (layer "F.Cu") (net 6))
 (segment (start 144.835 78.5) (end 144.835 78.300001) (width 0.25) (layer "F.Cu") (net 6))
 (via (at 151.2 82) (size 0.8) (drill 0.4) (layers "F.Cu" "B.Cu") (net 6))
 (via (at 151.2 79.3) (size 0.8) (drill 0.4) (layers "F.Cu" "B.Cu") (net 6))
 (segment (start 151.2 79.3) (end 151.2 82) (width 0.25) (layer "B.Cu") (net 6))
 (segment (start 144.68 82.5) (end 144.68 82.300001) (width 0.25) (layer "F.Cu") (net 7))
 (segment (start 152 80.7) (end 152 84) (width 0.25) (layer "F.Cu") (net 7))
 (segment (start 144.7 82.280001) (end 144.7 80.7) (width 0.25) (layer "F.Cu") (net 7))
 (segment (start 144.9 80.5) (end 148 80.5) (width 0.25) (layer "F.Cu") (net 7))
 (segment (start 148 80.5) (end 151.8 80.5) (width 0.25) (layer "F.Cu") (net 7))
 (segment (start 144.7 80.7) (end 144.9 80.5) (width 0.25) (layer "F.Cu") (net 7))
 (segment (start 151.8 80.5) (end 152 80.7) (width 0.25) (layer "F.Cu") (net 7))
 (segment (start 144.68 82.300001) (end 144.7 82.280001) (width 0.25) (layer "F.Cu") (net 7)))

